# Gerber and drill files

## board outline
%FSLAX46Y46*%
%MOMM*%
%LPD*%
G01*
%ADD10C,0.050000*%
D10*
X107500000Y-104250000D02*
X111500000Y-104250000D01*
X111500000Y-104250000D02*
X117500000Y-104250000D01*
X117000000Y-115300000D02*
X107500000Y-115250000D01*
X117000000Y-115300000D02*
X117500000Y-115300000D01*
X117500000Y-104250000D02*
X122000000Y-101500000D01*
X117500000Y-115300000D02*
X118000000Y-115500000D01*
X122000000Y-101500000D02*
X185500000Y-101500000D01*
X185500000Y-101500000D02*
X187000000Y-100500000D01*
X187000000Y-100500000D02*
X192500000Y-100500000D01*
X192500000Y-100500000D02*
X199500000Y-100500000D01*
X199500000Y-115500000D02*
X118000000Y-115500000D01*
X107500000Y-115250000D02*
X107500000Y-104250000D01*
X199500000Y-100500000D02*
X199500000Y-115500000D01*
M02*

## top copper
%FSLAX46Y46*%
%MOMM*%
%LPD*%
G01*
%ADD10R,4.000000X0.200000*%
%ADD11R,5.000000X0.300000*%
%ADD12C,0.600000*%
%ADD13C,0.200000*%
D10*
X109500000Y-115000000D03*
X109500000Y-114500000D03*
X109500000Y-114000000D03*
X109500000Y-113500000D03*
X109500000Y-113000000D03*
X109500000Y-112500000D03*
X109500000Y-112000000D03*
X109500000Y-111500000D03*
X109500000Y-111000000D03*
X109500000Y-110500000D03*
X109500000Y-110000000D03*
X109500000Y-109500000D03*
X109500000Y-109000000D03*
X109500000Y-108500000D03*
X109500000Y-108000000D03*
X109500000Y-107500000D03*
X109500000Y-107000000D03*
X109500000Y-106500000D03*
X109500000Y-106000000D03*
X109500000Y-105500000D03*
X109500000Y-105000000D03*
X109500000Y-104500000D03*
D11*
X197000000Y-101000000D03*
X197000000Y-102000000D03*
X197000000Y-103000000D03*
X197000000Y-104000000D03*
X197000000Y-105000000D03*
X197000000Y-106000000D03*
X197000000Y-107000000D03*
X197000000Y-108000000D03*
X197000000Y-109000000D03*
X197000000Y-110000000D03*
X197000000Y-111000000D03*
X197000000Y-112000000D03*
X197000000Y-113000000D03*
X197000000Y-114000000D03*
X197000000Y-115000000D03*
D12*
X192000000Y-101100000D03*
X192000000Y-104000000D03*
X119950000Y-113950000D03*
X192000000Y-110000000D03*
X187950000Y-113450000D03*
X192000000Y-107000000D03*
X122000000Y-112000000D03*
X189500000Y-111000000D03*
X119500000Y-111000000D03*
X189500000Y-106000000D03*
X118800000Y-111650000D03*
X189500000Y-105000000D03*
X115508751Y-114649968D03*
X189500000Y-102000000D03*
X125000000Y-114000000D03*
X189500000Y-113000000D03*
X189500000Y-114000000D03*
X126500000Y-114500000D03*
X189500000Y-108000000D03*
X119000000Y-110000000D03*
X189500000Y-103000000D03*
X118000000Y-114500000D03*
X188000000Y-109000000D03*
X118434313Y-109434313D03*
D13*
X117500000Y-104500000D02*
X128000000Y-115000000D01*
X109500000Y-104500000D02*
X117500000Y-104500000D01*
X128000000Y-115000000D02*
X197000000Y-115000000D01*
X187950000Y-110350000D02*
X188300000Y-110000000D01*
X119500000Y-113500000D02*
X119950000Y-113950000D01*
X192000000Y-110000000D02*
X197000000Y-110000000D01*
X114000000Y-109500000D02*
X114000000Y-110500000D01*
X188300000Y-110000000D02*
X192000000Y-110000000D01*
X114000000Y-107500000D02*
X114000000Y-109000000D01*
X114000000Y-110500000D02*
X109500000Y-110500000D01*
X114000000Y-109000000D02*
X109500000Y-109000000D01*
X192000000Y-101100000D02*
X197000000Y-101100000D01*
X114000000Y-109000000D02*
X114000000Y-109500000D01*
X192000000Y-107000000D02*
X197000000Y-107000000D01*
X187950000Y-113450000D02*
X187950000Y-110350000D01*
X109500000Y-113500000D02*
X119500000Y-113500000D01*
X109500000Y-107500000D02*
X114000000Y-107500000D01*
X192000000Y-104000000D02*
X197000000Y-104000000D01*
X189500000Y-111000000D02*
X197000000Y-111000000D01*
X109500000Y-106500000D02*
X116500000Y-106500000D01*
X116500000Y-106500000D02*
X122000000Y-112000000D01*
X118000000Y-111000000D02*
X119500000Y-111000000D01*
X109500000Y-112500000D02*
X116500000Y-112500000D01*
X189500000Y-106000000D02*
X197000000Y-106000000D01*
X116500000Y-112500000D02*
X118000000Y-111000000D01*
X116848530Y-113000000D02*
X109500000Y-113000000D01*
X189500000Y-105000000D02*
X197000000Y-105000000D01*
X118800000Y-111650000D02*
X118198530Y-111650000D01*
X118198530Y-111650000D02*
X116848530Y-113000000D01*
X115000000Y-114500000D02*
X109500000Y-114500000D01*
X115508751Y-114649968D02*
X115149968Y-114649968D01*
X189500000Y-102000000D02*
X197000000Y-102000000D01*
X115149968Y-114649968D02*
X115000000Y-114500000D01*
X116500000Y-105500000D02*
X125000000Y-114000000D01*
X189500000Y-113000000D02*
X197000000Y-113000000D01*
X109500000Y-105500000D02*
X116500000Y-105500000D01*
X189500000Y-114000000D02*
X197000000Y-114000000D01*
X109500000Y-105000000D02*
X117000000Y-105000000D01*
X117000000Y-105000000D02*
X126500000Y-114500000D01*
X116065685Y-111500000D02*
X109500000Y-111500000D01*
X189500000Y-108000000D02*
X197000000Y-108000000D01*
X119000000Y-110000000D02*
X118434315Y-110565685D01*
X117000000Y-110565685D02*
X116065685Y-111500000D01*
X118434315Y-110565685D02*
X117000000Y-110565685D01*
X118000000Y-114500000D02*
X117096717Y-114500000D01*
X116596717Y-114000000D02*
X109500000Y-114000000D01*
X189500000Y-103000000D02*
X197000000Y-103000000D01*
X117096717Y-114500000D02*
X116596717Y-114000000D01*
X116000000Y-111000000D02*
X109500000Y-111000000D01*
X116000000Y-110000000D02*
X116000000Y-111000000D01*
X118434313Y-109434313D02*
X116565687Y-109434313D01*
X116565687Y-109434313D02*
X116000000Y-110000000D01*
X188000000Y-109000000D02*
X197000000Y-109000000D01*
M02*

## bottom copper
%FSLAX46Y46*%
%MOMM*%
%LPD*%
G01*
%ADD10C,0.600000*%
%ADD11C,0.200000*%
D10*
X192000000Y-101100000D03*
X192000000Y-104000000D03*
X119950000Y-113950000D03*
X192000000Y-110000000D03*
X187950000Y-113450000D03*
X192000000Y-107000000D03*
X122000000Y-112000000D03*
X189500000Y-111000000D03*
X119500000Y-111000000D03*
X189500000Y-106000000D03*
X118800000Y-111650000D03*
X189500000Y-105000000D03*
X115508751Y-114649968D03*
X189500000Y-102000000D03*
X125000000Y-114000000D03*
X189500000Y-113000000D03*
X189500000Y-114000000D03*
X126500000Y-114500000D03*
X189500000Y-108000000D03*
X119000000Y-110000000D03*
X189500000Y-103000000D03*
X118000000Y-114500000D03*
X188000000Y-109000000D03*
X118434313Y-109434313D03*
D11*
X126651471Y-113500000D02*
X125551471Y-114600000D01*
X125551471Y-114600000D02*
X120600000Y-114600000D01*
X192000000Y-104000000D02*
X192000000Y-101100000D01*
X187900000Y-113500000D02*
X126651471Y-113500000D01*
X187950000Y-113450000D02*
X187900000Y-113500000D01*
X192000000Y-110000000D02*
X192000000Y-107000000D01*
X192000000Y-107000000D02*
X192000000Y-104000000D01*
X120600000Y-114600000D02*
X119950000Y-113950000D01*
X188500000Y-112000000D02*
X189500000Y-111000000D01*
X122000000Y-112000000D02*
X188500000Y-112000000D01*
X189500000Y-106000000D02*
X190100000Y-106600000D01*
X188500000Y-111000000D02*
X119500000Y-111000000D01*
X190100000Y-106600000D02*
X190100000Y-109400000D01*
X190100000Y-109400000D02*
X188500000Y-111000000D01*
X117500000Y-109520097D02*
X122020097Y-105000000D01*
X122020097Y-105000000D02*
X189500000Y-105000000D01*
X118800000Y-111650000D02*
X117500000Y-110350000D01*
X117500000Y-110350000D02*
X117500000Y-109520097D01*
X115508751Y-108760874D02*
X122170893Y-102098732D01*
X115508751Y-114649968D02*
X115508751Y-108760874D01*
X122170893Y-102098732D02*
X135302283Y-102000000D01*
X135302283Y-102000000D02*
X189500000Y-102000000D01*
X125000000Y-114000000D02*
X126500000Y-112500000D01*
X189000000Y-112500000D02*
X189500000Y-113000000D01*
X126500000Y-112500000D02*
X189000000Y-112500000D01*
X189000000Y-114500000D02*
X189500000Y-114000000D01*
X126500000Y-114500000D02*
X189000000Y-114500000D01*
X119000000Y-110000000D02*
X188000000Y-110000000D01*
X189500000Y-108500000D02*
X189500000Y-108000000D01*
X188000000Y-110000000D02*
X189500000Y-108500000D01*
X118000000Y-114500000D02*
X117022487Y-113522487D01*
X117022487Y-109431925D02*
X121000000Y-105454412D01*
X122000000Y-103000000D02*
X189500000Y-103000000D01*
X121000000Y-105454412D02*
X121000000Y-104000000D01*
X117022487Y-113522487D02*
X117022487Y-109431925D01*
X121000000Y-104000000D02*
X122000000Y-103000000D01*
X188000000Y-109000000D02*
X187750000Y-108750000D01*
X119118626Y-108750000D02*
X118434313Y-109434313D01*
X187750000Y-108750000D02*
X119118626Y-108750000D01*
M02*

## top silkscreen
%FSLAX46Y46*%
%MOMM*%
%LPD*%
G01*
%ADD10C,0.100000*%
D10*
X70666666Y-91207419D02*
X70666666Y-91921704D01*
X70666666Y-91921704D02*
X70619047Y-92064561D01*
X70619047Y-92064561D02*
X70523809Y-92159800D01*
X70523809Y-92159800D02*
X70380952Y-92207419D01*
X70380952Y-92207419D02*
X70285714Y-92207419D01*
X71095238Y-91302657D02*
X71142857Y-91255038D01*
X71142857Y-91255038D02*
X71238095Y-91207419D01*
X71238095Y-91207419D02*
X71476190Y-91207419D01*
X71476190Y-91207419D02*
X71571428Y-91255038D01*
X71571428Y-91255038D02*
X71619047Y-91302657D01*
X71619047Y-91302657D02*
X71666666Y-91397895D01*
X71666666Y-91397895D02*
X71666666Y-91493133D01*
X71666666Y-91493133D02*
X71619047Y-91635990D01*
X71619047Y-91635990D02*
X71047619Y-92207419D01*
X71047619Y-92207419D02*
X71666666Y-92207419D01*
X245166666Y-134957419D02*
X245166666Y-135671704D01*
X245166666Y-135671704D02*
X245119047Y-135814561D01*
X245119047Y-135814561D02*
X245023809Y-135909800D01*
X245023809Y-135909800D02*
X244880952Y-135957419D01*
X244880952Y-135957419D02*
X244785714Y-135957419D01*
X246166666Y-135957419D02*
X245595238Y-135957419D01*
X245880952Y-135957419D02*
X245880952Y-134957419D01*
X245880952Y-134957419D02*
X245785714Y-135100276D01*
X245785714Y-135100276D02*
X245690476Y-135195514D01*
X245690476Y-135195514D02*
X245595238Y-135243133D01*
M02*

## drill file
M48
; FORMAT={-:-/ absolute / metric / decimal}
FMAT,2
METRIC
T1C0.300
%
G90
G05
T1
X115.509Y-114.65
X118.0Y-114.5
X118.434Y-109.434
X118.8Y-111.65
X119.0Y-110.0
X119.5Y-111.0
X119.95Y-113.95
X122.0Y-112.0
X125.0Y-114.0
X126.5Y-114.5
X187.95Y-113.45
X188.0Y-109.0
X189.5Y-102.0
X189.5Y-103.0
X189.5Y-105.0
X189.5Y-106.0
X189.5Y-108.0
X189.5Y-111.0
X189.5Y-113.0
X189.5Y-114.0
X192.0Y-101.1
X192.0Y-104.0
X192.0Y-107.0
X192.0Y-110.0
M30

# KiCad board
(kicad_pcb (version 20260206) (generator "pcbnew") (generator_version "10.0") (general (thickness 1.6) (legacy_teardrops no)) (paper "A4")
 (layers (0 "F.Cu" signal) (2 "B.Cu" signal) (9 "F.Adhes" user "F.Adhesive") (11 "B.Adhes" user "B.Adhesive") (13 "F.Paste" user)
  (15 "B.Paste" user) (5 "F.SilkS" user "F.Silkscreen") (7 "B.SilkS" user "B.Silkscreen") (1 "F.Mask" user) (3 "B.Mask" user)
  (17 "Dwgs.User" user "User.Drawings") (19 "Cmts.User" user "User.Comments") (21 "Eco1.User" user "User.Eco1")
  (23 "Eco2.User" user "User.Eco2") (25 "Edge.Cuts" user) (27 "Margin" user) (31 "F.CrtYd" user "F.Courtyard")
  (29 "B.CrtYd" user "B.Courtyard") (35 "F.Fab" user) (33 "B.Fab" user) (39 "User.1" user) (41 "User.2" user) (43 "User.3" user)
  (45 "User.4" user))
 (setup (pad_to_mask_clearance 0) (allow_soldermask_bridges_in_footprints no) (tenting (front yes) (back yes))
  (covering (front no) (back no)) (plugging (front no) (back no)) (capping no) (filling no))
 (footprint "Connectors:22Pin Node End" (layer "F.Cu") (at 109.5 109.75 180)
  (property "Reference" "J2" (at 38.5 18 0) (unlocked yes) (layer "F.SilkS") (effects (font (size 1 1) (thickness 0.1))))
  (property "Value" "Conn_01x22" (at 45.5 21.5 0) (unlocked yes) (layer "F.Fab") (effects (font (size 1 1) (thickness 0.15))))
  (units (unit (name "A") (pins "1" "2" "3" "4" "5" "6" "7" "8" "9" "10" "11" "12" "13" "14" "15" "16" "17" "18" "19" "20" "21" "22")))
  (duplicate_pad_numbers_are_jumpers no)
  (fp_line (start 2 -5.5) (end 2 5.5) (stroke (width 0.05) (type default)) (layer "Edge.Cuts"))
  (pad "1" smd rect (at 0 -5.25 180) (size 4 0.2) (layers "F.Cu" "F.Mask" "F.Paste") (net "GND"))
  (pad "2" smd rect (at 0 -4.75 180) (size 4 0.2) (layers "F.Cu" "F.Mask" "F.Paste") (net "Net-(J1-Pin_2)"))
  (pad "3" smd rect (at 0 -4.25 180) (size 4 0.2) (layers "F.Cu" "F.Mask" "F.Paste") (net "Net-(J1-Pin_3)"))
  (pad "4" smd rect (at 0 -3.75 180) (size 4 0.2) (layers "F.Cu" "F.Mask" "F.Paste") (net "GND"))
  (pad "5" smd rect (at 0 -3.25 180) (size 4 0.2) (layers "F.Cu" "F.Mask" "F.Paste") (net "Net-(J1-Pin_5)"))
  (pad "6" smd rect (at 0 -2.75 180) (size 4 0.2) (layers "F.Cu" "F.Mask" "F.Paste") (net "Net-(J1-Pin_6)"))
  (pad "7" smd rect (at 0 -2.25 180) (size 4 0.2) (layers "F.Cu" "F.Mask" "F.Paste") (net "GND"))
  (pad "8" smd rect (at 0 -1.75 180) (size 4 0.2) (layers "F.Cu" "F.Mask" "F.Paste") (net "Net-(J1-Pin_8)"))
  (pad "9" smd rect (at 0 -1.25 180) (size 4 0.2) (layers "F.Cu" "F.Mask" "F.Paste") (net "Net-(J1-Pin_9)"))
  (pad "10" smd rect (at 0 -0.75 180) (size 4 0.2) (layers "F.Cu" "F.Mask" "F.Paste") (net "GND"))
  (pad "11" smd rect (at 0 -0.25 180) (size 4 0.2) (layers "F.Cu" "F.Mask" "F.Paste") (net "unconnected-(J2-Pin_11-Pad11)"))
  (pad "12" smd rect (at 0 0.25 180) (size 4 0.2) (layers "F.Cu" "F.Mask" "F.Paste") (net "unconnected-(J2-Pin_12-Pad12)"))
  (pad "13" smd rect (at 0 0.75 180) (size 4 0.2) (layers "F.Cu" "F.Mask" "F.Paste") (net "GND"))
  (pad "14" smd rect (at 0 1.25 180) (size 4 0.2) (layers "F.Cu" "F.Mask" "F.Paste") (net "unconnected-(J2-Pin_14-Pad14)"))
  (pad "15" smd rect (at 0 1.75 180) (size 4 0.2) (layers "F.Cu" "F.Mask" "F.Paste") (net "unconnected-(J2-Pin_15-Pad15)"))
  (pad "16" smd rect (at 0 2.25 180) (size 4 0.2) (layers "F.Cu" "F.Mask" "F.Paste") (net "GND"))
  (pad "17" smd rect (at 0 2.75 180) (size 4 0.2) (layers "F.Cu" "F.Mask" "F.Paste") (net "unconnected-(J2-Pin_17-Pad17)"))
  (pad "18" smd rect (at 0 3.25 180) (size 4 0.2) (layers "F.Cu" "F.Mask" "F.Paste") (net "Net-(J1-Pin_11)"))
  (pad "19" smd rect (at 0 3.75 180) (size 4 0.2) (layers "F.Cu" "F.Mask" "F.Paste") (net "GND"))
  (pad "20" smd rect (at 0 4.25 180) (size 4 0.2) (layers "F.Cu" "F.Mask" "F.Paste") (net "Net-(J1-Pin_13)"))
  (pad "21" smd rect (at 0 4.75 180) (size 4 0.2) (layers "F.Cu" "F.Mask" "F.Paste") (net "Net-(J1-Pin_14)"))
  (pad "22" smd rect (at 0 5.25 180) (size 4 0.2) (layers "F.Cu" "F.Mask" "F.Paste") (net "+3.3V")))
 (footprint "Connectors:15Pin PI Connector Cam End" (layer "F.Cu") (at 197 108)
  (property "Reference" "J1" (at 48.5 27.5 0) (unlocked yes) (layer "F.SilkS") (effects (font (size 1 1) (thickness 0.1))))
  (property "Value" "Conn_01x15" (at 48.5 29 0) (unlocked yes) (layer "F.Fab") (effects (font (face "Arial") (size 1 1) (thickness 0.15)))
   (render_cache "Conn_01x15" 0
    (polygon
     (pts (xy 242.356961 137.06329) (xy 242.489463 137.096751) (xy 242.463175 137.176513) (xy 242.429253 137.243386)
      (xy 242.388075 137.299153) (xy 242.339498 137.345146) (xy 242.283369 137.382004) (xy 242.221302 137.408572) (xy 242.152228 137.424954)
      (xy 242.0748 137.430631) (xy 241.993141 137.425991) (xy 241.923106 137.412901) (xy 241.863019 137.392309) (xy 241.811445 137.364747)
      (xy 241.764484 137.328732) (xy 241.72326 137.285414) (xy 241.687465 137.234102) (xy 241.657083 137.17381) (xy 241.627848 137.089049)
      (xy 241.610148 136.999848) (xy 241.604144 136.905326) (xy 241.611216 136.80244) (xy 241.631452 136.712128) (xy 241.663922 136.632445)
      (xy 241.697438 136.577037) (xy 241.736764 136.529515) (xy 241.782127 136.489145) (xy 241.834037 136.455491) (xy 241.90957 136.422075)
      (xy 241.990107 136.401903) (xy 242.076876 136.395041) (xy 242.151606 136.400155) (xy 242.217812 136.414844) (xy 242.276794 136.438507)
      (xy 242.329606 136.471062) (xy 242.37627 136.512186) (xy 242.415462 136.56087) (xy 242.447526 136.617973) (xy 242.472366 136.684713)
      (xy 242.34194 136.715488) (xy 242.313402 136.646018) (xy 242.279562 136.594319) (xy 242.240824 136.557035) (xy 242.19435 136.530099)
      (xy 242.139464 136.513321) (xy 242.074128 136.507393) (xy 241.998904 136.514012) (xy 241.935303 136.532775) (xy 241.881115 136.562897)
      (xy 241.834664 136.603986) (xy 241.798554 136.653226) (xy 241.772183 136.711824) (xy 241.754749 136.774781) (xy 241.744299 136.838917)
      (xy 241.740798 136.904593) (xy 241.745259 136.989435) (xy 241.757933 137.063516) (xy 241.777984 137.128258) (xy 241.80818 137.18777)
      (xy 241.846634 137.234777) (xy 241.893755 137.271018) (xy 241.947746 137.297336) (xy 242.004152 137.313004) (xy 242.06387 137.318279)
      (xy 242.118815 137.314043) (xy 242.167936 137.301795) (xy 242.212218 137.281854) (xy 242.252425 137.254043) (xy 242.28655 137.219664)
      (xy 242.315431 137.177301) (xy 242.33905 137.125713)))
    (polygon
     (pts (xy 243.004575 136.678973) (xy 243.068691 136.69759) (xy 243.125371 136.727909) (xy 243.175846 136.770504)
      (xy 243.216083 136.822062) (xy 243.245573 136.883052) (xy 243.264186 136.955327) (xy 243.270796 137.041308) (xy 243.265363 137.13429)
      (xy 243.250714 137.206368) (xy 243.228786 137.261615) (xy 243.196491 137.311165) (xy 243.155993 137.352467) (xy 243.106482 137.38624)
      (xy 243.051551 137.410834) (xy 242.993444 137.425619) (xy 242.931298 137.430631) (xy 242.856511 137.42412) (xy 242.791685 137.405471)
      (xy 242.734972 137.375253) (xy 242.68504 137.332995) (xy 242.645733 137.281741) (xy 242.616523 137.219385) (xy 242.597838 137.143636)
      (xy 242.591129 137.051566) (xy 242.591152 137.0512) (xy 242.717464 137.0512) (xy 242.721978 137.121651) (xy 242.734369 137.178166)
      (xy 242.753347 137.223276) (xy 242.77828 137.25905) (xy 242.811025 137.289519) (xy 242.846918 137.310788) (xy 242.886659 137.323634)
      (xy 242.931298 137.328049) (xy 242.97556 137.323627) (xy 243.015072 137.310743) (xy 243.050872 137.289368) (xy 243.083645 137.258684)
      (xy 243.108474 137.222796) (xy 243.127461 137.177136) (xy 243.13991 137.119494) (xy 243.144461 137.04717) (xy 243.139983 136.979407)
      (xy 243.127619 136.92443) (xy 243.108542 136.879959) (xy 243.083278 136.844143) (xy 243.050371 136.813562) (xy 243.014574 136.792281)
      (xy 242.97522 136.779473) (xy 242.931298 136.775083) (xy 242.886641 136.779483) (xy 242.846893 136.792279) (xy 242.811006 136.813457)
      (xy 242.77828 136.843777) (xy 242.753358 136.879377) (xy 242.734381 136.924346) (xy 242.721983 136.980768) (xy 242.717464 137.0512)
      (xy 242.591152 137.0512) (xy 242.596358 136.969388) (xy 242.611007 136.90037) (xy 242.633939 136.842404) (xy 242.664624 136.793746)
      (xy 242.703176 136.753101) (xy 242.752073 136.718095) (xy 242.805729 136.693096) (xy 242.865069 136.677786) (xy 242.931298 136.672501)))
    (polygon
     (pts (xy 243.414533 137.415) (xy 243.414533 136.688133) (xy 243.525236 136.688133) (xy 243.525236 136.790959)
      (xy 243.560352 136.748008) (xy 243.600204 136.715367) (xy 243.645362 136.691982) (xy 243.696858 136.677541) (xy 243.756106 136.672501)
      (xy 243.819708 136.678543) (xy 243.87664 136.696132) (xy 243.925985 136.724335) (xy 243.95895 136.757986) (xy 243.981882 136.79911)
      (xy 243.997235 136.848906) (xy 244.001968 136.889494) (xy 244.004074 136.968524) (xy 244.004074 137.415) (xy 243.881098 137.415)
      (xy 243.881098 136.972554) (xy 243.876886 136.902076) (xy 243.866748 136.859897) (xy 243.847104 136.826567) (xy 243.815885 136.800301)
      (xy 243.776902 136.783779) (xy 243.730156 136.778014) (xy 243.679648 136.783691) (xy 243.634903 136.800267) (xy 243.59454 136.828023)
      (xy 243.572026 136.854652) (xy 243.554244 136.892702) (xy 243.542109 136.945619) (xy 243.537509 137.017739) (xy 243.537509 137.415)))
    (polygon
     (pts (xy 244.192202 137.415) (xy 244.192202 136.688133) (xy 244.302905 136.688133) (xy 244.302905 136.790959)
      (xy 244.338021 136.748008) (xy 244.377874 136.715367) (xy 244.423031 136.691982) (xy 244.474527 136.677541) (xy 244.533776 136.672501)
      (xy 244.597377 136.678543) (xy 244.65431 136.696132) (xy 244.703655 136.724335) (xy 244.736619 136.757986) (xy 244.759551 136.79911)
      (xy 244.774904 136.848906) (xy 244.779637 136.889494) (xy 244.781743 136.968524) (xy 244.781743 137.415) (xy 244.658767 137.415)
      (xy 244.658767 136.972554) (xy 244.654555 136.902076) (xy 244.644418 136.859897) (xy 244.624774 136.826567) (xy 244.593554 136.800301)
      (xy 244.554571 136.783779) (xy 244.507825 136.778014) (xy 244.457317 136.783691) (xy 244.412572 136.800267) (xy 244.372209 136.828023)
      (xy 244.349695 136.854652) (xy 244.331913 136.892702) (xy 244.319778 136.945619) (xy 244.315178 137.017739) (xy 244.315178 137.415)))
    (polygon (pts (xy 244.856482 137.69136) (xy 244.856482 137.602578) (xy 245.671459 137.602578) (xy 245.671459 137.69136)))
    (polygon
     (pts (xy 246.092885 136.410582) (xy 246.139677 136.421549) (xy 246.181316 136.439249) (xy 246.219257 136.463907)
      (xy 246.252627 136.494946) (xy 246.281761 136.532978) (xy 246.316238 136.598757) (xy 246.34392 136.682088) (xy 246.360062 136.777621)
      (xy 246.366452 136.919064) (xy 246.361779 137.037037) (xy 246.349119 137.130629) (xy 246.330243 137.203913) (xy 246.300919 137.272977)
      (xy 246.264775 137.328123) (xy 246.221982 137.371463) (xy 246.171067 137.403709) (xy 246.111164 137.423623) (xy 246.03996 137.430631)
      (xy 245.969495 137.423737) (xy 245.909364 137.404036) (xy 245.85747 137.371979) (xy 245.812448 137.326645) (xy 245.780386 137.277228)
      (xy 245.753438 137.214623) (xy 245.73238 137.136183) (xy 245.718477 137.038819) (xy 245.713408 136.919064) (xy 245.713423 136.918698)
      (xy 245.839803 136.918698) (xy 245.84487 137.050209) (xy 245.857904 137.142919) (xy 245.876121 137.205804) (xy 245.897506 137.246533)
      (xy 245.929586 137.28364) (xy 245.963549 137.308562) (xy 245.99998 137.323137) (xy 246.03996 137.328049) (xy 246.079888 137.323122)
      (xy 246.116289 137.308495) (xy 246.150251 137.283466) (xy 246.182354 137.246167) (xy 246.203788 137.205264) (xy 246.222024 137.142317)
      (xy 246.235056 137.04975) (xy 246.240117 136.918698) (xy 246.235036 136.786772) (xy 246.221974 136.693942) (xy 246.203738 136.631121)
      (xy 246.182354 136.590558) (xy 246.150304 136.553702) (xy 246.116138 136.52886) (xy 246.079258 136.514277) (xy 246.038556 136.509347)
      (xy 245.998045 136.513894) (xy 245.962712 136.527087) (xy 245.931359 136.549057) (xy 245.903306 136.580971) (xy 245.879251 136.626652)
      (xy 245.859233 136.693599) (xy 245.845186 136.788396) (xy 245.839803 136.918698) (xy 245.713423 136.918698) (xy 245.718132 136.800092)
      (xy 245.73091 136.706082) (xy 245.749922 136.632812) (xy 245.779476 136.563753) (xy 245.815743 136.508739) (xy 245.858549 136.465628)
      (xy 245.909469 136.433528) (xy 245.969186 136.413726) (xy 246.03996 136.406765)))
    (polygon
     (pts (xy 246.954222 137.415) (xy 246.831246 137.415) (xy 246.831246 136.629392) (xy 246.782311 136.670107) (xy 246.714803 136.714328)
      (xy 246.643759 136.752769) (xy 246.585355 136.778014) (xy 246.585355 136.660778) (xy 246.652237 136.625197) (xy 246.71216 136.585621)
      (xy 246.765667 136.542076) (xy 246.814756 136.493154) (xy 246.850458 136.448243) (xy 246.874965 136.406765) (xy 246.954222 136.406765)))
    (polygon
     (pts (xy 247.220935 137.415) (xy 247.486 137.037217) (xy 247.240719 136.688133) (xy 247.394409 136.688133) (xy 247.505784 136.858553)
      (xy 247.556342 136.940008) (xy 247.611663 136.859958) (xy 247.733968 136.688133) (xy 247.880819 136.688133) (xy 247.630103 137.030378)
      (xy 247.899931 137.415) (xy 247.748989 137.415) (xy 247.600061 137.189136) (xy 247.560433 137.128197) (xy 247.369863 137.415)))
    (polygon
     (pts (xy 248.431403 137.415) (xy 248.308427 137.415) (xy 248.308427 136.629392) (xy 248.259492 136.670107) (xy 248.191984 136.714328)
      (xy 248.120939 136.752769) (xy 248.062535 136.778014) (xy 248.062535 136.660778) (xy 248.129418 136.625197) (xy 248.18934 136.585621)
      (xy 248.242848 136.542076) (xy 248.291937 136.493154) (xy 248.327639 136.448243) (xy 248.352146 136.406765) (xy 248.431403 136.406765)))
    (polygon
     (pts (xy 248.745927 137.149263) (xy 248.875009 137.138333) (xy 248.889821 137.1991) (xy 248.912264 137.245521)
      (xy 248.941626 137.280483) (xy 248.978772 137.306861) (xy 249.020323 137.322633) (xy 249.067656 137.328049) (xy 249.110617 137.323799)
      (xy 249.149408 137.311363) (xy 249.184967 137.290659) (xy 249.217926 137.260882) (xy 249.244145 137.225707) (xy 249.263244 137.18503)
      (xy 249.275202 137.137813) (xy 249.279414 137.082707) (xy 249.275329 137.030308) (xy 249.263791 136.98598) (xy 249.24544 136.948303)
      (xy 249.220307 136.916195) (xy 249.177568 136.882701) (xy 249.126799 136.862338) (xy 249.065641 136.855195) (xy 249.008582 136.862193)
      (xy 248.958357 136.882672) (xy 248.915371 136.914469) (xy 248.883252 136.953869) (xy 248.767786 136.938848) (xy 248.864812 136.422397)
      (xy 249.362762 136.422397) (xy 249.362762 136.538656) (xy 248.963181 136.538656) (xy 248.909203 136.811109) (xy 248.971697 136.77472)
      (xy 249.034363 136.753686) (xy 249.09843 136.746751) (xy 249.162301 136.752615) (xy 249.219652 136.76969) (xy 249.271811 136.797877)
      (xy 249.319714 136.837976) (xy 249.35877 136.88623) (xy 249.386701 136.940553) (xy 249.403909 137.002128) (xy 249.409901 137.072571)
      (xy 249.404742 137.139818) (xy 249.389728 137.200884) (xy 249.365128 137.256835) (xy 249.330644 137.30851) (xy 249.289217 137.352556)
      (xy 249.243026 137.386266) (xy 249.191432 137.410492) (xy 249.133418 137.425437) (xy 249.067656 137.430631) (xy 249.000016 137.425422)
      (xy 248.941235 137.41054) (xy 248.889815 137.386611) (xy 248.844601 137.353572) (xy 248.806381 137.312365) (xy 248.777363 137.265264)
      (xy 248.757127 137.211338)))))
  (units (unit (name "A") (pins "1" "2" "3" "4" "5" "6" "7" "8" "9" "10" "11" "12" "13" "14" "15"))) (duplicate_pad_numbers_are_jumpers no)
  (fp_line (start 2.5 -7.5) (end 2.5 7.5) (stroke (width 0.05) (type default)) (layer "Edge.Cuts"))
  (pad "1" smd rect (at 0 -7) (size 5 0.3) (layers "F.Cu" "F.Mask" "F.Paste") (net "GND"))
  (pad "2" smd rect (at 0 -6) (size 5 0.3) (layers "F.Cu" "F.Mask" "F.Paste") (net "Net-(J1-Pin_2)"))
  (pad "3" smd rect (at 0 -5) (size 5 0.3) (layers "F.Cu" "F.Mask" "F.Paste") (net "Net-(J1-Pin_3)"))
  (pad "4" smd rect (at 0 -4) (size 5 0.3) (layers "F.Cu" "F.Mask" "F.Paste") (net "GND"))
  (pad "5" smd rect (at 0 -3) (size 5 0.3) (layers "F.Cu" "F.Mask" "F.Paste") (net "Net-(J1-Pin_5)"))
  (pad "6" smd rect (at 0 -2) (size 5 0.3) (layers "F.Cu" "F.Mask" "F.Paste") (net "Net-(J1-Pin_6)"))
  (pad "7" smd rect (at 0 -1) (size 5 0.3) (layers "F.Cu" "F.Mask" "F.Paste") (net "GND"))
  (pad "8" smd rect (at 0 0) (size 5 0.3) (layers "F.Cu" "F.Mask" "F.Paste") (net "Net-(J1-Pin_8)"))
  (pad "9" smd rect (at 0 1) (size 5 0.3) (layers "F.Cu" "F.Mask" "F.Paste") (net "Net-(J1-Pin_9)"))
  (pad "10" smd rect (at 0 2) (size 5 0.3) (layers "F.Cu" "F.Mask" "F.Paste") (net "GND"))
  (pad "11" smd rect (at 0 3) (size 5 0.3) (layers "F.Cu" "F.Mask" "F.Paste") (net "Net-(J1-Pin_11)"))
  (pad "12" smd rect (at 0 4) (size 5 0.3) (layers "F.Cu" "F.Mask" "F.Paste") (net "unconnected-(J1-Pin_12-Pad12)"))
  (pad "13" smd rect (at 0 5) (size 5 0.3) (layers "F.Cu" "F.Mask" "F.Paste") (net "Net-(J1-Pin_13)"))
  (pad "14" smd rect (at 0 6) (size 5 0.3) (layers "F.Cu" "F.Mask" "F.Paste") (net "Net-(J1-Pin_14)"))
  (pad "15" smd rect (at 0 7) (size 5 0.3) (layers "F.Cu" "F.Mask" "F.Paste") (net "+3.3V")))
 (gr_line (start 107.5 104.25) (end 111.5 104.25) (stroke (width 0.05) (type default)) (layer "Edge.Cuts"))
 (gr_line (start 111.5 104.25) (end 117.5 104.25) (stroke (width 0.05) (type default)) (layer "Edge.Cuts"))
 (gr_line (start 117 115.3) (end 107.5 115.25) (stroke (width 0.05) (type default)) (layer "Edge.Cuts"))
 (gr_line (start 117 115.3) (end 117.5 115.3) (stroke (width 0.05) (type default)) (layer "Edge.Cuts"))
 (gr_line (start 117.5 104.25) (end 122 101.5) (stroke (width 0.05) (type default)) (layer "Edge.Cuts"))
 (gr_line (start 117.5 115.3) (end 118 115.5) (stroke (width 0.05) (type default)) (layer "Edge.Cuts"))
 (gr_line (start 122 101.5) (end 185.5 101.5) (stroke (width 0.05) (type default)) (layer "Edge.Cuts"))
 (gr_line (start 185.5 101.5) (end 187 100.5) (stroke (width 0.05) (type default)) (layer "Edge.Cuts"))
 (gr_line (start 187 100.5) (end 192.5 100.5) (stroke (width 0.05) (type default)) (layer "Edge.Cuts"))
 (gr_line (start 192.5 100.5) (end 199.5 100.5) (stroke (width 0.05) (type default)) (layer "Edge.Cuts"))
 (gr_line (start 199.5 115.5) (end 118 115.5) (stroke (width 0.05) (type default)) (layer "Edge.Cuts"))
 (segment (start 117.5 104.5) (end 128 115) (width 0.2) (layer "F.Cu") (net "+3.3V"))
 (segment (start 109.5 104.5) (end 117.5 104.5) (width 0.2) (layer "F.Cu") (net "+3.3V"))
 (segment (start 128 115) (end 197 115) (width 0.2) (layer "F.Cu") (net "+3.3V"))
 (segment (start 187.95 110.35) (end 188.3 110) (width 0.2) (layer "F.Cu") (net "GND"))
 (segment (start 119.5 113.5) (end 119.95 113.95) (width 0.2) (layer "F.Cu") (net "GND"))
 (segment (start 192 110) (end 197 110) (width 0.2) (layer "F.Cu") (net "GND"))
 (segment (start 114 109.5) (end 114 110.5) (width 0.2) (layer "F.Cu") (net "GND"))
 (segment (start 188.3 110) (end 192 110) (width 0.2) (layer "F.Cu") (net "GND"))
 (segment (start 114 107.5) (end 114 109) (width 0.2) (layer "F.Cu") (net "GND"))
 (segment (start 114 110.5) (end 109.5 110.5) (width 0.2) (layer "F.Cu") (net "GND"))
 (segment (start 114 109) (end 109.5 109) (width 0.2) (layer "F.Cu") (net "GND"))
 (segment (start 192 101.1) (end 197 101.1) (width 0.2) (layer "F.Cu") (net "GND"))
 (segment (start 114 109) (end 114 109.5) (width 0.2) (layer "F.Cu") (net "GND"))
 (segment (start 192 107) (end 197 107) (width 0.2) (layer "F.Cu") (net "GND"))
 (segment (start 187.95 113.45) (end 187.95 110.35) (width 0.2) (layer "F.Cu") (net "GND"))
 (segment (start 109.5 113.5) (end 119.5 113.5) (width 0.2) (layer "F.Cu") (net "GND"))
 (segment (start 109.5 107.5) (end 114 107.5) (width 0.2) (layer "F.Cu") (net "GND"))
 (segment (start 192 104) (end 197 104) (width 0.2) (layer "F.Cu") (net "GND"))
 (via (at 192 101.1) (size 0.6) (drill 0.3) (layers "F.Cu" "B.Cu") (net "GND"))
 (via (at 192 104) (size 0.6) (drill 0.3) (layers "F.Cu" "B.Cu") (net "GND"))
 (via (at 119.95 113.95) (size 0.6) (drill 0.3) (layers "F.Cu" "B.Cu") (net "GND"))
 (via (at 192 110) (size 0.6) (drill 0.3) (layers "F.Cu" "B.Cu") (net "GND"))
 (via (at 187.95 113.45) (size 0.6) (drill 0.3) (layers "F.Cu" "B.Cu") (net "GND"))
 (via (at 192 107) (size 0.6) (drill 0.3) (layers "F.Cu" "B.Cu") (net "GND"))
 (segment (start 126.651471 113.5) (end 125.551471 114.6) (width 0.2) (layer "B.Cu") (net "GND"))
 (segment (start 125.551471 114.6) (end 120.6 114.6) (width 0.2) (layer "B.Cu") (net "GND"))
 (segment (start 192 104) (end 192 101.1) (width 0.2) (layer "B.Cu") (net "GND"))
 (segment (start 187.9 113.5) (end 126.651471 113.5) (width 0.2) (layer "B.Cu") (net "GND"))
 (segment (start 187.95 113.45) (end 187.9 113.5) (width 0.2) (layer "B.Cu") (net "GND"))
 (segment (start 192 110) (end 192 107) (width 0.2) (layer "B.Cu") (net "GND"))
 (segment (start 192 107) (end 192 104) (width 0.2) (layer "B.Cu") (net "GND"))
 (segment (start 120.6 114.6) (end 119.95 113.95) (width 0.2) (layer "B.Cu") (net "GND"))
 (segment (start 189.5 111) (end 197 111) (width 0.2) (layer "F.Cu") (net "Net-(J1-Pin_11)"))
 (segment (start 109.5 106.5) (end 116.5 106.5) (width 0.2) (layer "F.Cu") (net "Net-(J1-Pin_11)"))
 (segment (start 116.5 106.5) (end 122 112) (width 0.2) (layer "F.Cu") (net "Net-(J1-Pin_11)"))
 (via (at 122 112) (size 0.6) (drill 0.3) (layers "F.Cu" "B.Cu") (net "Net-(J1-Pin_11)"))
 (via (at 189.5 111) (size 0.6) (drill 0.3) (layers "F.Cu" "B.Cu") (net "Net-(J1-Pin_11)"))
 (segment (start 188.5 112) (end 189.5 111) (width 0.2) (layer "B.Cu") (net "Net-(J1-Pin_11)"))
 (segment (start 122 112) (end 188.5 112) (width 0.2) (layer "B.Cu") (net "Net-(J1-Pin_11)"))
 (segment (start 118 111) (end 119.5 111) (width 0.2) (layer "F.Cu") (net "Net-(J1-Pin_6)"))
 (segment (start 109.5 112.5) (end 116.5 112.5) (width 0.2) (layer "F.Cu") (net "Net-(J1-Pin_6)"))
 (segment (start 189.5 106) (end 197 106) (width 0.2) (layer "F.Cu") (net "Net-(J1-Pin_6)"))
 (segment (start 116.5 112.5) (end 118 111) (width 0.2) (layer "F.Cu") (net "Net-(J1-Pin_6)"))
 (via (at 119.5 111) (size 0.6) (drill 0.3) (layers "F.Cu" "B.Cu") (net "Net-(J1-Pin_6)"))
 (via (at 189.5 106) (size 0.6) (drill 0.3) (layers "F.Cu" "B.Cu") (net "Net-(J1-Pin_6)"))
 (segment (start 189.5 106) (end 190.1 106.6) (width 0.2) (layer "B.Cu") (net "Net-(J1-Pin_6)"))
 (segment (start 188.5 111) (end 119.5 111) (width 0.2) (layer "B.Cu") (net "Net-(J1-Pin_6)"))
 (segment (start 190.1 106.6) (end 190.1 109.4) (width 0.2) (layer "B.Cu") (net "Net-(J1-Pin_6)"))
 (segment (start 190.1 109.4) (end 188.5 111) (width 0.2) (layer "B.Cu") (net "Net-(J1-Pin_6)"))
 (segment (start 116.84853 113) (end 109.5 113) (width 0.2) (layer "F.Cu") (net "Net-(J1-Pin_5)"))
 (segment (start 189.5 105) (end 197 105) (width 0.2) (layer "F.Cu") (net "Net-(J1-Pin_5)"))
 (segment (start 118.8 111.65) (end 118.19853 111.65) (width 0.2) (layer "F.Cu") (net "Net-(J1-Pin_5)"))
 (segment (start 118.19853 111.65) (end 116.84853 113) (width 0.2) (layer "F.Cu") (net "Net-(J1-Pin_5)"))
 (via (at 118.8 111.65) (size 0.6) (drill 0.3) (layers "F.Cu" "B.Cu") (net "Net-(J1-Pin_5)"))
 (via (at 189.5 105) (size 0.6) (drill 0.3) (layers "F.Cu" "B.Cu") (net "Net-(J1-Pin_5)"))
 (segment (start 117.5 109.520097) (end 122.020097 105) (width 0.2) (layer "B.Cu") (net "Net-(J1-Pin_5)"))
 (segment (start 122.020097 105) (end 189.5 105) (width 0.2) (layer "B.Cu") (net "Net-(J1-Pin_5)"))
 (segment (start 118.8 111.65) (end 117.5 110.35) (width 0.2) (layer "B.Cu") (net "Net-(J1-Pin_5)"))
 (segment (start 117.5 110.35) (end 117.5 109.520097) (width 0.2) (layer "B.Cu") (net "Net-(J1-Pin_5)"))
 (segment (start 115 114.5) (end 109.5 114.5) (width 0.2) (layer "F.Cu") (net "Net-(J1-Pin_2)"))
 (segment (start 115.508751 114.649968) (end 115.149968 114.649968) (width 0.2) (layer "F.Cu") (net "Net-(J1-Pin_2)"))
 (segment (start 189.5 102) (end 197 102) (width 0.2) (layer "F.Cu") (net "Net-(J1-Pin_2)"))
 (segment (start 115.149968 114.649968) (end 115 114.5) (width 0.2) (layer "F.Cu") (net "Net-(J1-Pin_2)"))
 (via (at 115.508751 114.649968) (size 0.6) (drill 0.3) (layers "F.Cu" "B.Cu") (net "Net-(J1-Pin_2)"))
 (via (at 189.5 102) (size 0.6) (drill 0.3) (layers "F.Cu" "B.Cu") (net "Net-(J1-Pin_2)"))
 (segment (start 115.508751 108.760874) (end 122.170893 102.098732) (width 0.2) (layer "B.Cu") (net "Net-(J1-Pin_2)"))
 (segment (start 115.508751 114.649968) (end 115.508751 108.760874) (width 0.2) (layer "B.Cu") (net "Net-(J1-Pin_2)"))
 (segment (start 122.170893 102.098732) (end 135.302283 102) (width 0.2) (layer "B.Cu") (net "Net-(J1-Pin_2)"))
 (segment (start 135.302283 102) (end 189.5 102) (width 0.2) (layer "B.Cu") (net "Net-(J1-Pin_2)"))
 (segment (start 116.5 105.5) (end 125 114) (width 0.2) (layer "F.Cu") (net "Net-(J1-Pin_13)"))
 (segment (start 189.5 113) (end 197 113) (width 0.2) (layer "F.Cu") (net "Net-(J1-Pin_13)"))
 (segment (start 109.5 105.5) (end 116.5 105.5) (width 0.2) (layer "F.Cu") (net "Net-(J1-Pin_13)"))
 (via (at 125 114) (size 0.6) (drill 0.3) (layers "F.Cu" "B.Cu") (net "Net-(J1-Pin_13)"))
 (via (at 189.5 113) (size 0.6) (drill 0.3) (layers "F.Cu" "B.Cu") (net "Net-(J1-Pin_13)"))
 (segment (start 125 114) (end 126.5 112.5) (width 0.2) (layer "B.Cu") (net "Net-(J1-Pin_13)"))
 (segment (start 189 112.5) (end 189.5 113) (width 0.2) (layer "B.Cu") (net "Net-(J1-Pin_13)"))
 (segment (start 126.5 112.5) (end 189 112.5) (width 0.2) (layer "B.Cu") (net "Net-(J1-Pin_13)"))
 (segment (start 189.5 114) (end 197 114) (width 0.2) (layer "F.Cu") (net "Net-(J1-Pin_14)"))
 (segment (start 109.5 105) (end 117 105) (width 0.2) (layer "F.Cu") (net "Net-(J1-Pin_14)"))
 (segment (start 117 105) (end 126.5 114.5) (width 0.2) (layer "F.Cu") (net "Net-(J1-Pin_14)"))
 (via (at 189.5 114) (size 0.6) (drill 0.3) (layers "F.Cu" "B.Cu") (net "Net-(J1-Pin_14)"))
 (via (at 126.5 114.5) (size 0.6) (drill 0.3) (layers "F.Cu" "B.Cu") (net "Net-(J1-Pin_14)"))
 (segment (start 189 114.5) (end 189.5 114) (width 0.2) (layer "B.Cu") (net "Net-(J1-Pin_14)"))
 (segment (start 126.5 114.5) (end 189 114.5) (width 0.2) (layer "B.Cu") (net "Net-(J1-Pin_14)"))
 (segment (start 116.065685 111.5) (end 109.5 111.5) (width 0.2) (layer "F.Cu") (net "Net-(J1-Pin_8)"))
 (segment (start 189.5 108) (end 197 108) (width 0.2) (layer "F.Cu") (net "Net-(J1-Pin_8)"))
 (segment (start 119 110) (end 118.434315 110.565685) (width 0.2) (layer "F.Cu") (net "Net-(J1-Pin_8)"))
 (segment (start 117 110.565685) (end 116.065685 111.5) (width 0.2) (layer "F.Cu") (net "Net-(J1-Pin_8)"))
 (segment (start 118.434315 110.565685) (end 117 110.565685) (width 0.2) (layer "F.Cu") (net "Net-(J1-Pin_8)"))
 (via (at 189.5 108) (size 0.6) (drill 0.3) (layers "F.Cu" "B.Cu") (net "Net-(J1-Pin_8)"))
 (via (at 119 110) (size 0.6) (drill 0.3) (layers "F.Cu" "B.Cu") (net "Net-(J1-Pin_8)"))
 (segment (start 119 110) (end 188 110) (width 0.2) (layer "B.Cu") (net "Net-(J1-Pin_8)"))
 (segment (start 189.5 108.5) (end 189.5 108) (width 0.2) (layer "B.Cu") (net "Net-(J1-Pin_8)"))
 (segment (start 188 110) (end 189.5 108.5) (width 0.2) (layer "B.Cu") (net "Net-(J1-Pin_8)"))
 (segment (start 118 114.5) (end 117.096717 114.5) (width 0.2) (layer "F.Cu") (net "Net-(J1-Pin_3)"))
 (segment (start 116.596717 114) (end 109.5 114) (width 0.2) (layer "F.Cu") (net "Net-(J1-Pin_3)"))
 (segment (start 189.5 103) (end 197 103) (width 0.2) (layer "F.Cu") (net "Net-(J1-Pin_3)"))
 (segment (start 117.096717 114.5) (end 116.596717 114) (width 0.2) (layer "F.Cu") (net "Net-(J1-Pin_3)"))
 (via (at 189.5 103) (size 0.6) (drill 0.3) (layers "F.Cu" "B.Cu") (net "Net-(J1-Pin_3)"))
 (via (at 118 114.5) (size 0.6) (drill 0.3) (layers "F.Cu" "B.Cu") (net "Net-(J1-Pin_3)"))
 (segment (start 118 114.5) (end 117.022487 113.522487) (width 0.2) (layer "B.Cu") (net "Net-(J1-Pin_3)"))
 (segment (start 117.022487 109.431925) (end 121 105.454412) (width 0.2) (layer "B.Cu") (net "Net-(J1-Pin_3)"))
 (segment (start 122 103) (end 189.5 103) (width 0.2) (layer "B.Cu") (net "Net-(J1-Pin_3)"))
 (segment (start 121 105.454412) (end 121 104) (width 0.2) (layer "B.Cu") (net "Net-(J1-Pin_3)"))
 (segment (start 117.022487 113.522487) (end 117.022487 109.431925) (width 0.2) (layer "B.Cu") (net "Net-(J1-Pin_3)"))
 (segment (start 121 104) (end 122 103) (width 0.2) (layer "B.Cu") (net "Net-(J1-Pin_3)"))
 (segment (start 116 111) (end 109.5 111) (width 0.2) (layer "F.Cu") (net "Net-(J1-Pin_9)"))
 (segment (start 116 110) (end 116 111) (width 0.2) (layer "F.Cu") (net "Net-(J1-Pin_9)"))
 (segment (start 118.434313 109.434313) (end 116.565687 109.434313) (width 0.2) (layer "F.Cu") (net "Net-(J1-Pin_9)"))
 (segment (start 116.565687 109.434313) (end 116 110) (width 0.2) (layer "F.Cu") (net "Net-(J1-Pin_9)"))
 (segment (start 188 109) (end 197 109) (width 0.2) (layer "F.Cu") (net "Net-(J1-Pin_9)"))
 (via (at 188 109) (size 0.6) (drill 0.3) (layers "F.Cu" "B.Cu") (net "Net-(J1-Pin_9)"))
 (via (at 118.434313 109.434313) (size 0.6) (drill 0.3) (layers "F.Cu" "B.Cu") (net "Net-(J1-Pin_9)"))
 (segment (start 188 109) (end 187.75 108.75) (width 0.2) (layer "B.Cu") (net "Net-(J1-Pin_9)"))
 (segment (start 119.118626 108.75) (end 118.434313 109.434313) (width 0.2) (layer "B.Cu") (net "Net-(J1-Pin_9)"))
 (segment (start 187.75 108.75) (end 119.118626 108.75) (width 0.2) (layer "B.Cu") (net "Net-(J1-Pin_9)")))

